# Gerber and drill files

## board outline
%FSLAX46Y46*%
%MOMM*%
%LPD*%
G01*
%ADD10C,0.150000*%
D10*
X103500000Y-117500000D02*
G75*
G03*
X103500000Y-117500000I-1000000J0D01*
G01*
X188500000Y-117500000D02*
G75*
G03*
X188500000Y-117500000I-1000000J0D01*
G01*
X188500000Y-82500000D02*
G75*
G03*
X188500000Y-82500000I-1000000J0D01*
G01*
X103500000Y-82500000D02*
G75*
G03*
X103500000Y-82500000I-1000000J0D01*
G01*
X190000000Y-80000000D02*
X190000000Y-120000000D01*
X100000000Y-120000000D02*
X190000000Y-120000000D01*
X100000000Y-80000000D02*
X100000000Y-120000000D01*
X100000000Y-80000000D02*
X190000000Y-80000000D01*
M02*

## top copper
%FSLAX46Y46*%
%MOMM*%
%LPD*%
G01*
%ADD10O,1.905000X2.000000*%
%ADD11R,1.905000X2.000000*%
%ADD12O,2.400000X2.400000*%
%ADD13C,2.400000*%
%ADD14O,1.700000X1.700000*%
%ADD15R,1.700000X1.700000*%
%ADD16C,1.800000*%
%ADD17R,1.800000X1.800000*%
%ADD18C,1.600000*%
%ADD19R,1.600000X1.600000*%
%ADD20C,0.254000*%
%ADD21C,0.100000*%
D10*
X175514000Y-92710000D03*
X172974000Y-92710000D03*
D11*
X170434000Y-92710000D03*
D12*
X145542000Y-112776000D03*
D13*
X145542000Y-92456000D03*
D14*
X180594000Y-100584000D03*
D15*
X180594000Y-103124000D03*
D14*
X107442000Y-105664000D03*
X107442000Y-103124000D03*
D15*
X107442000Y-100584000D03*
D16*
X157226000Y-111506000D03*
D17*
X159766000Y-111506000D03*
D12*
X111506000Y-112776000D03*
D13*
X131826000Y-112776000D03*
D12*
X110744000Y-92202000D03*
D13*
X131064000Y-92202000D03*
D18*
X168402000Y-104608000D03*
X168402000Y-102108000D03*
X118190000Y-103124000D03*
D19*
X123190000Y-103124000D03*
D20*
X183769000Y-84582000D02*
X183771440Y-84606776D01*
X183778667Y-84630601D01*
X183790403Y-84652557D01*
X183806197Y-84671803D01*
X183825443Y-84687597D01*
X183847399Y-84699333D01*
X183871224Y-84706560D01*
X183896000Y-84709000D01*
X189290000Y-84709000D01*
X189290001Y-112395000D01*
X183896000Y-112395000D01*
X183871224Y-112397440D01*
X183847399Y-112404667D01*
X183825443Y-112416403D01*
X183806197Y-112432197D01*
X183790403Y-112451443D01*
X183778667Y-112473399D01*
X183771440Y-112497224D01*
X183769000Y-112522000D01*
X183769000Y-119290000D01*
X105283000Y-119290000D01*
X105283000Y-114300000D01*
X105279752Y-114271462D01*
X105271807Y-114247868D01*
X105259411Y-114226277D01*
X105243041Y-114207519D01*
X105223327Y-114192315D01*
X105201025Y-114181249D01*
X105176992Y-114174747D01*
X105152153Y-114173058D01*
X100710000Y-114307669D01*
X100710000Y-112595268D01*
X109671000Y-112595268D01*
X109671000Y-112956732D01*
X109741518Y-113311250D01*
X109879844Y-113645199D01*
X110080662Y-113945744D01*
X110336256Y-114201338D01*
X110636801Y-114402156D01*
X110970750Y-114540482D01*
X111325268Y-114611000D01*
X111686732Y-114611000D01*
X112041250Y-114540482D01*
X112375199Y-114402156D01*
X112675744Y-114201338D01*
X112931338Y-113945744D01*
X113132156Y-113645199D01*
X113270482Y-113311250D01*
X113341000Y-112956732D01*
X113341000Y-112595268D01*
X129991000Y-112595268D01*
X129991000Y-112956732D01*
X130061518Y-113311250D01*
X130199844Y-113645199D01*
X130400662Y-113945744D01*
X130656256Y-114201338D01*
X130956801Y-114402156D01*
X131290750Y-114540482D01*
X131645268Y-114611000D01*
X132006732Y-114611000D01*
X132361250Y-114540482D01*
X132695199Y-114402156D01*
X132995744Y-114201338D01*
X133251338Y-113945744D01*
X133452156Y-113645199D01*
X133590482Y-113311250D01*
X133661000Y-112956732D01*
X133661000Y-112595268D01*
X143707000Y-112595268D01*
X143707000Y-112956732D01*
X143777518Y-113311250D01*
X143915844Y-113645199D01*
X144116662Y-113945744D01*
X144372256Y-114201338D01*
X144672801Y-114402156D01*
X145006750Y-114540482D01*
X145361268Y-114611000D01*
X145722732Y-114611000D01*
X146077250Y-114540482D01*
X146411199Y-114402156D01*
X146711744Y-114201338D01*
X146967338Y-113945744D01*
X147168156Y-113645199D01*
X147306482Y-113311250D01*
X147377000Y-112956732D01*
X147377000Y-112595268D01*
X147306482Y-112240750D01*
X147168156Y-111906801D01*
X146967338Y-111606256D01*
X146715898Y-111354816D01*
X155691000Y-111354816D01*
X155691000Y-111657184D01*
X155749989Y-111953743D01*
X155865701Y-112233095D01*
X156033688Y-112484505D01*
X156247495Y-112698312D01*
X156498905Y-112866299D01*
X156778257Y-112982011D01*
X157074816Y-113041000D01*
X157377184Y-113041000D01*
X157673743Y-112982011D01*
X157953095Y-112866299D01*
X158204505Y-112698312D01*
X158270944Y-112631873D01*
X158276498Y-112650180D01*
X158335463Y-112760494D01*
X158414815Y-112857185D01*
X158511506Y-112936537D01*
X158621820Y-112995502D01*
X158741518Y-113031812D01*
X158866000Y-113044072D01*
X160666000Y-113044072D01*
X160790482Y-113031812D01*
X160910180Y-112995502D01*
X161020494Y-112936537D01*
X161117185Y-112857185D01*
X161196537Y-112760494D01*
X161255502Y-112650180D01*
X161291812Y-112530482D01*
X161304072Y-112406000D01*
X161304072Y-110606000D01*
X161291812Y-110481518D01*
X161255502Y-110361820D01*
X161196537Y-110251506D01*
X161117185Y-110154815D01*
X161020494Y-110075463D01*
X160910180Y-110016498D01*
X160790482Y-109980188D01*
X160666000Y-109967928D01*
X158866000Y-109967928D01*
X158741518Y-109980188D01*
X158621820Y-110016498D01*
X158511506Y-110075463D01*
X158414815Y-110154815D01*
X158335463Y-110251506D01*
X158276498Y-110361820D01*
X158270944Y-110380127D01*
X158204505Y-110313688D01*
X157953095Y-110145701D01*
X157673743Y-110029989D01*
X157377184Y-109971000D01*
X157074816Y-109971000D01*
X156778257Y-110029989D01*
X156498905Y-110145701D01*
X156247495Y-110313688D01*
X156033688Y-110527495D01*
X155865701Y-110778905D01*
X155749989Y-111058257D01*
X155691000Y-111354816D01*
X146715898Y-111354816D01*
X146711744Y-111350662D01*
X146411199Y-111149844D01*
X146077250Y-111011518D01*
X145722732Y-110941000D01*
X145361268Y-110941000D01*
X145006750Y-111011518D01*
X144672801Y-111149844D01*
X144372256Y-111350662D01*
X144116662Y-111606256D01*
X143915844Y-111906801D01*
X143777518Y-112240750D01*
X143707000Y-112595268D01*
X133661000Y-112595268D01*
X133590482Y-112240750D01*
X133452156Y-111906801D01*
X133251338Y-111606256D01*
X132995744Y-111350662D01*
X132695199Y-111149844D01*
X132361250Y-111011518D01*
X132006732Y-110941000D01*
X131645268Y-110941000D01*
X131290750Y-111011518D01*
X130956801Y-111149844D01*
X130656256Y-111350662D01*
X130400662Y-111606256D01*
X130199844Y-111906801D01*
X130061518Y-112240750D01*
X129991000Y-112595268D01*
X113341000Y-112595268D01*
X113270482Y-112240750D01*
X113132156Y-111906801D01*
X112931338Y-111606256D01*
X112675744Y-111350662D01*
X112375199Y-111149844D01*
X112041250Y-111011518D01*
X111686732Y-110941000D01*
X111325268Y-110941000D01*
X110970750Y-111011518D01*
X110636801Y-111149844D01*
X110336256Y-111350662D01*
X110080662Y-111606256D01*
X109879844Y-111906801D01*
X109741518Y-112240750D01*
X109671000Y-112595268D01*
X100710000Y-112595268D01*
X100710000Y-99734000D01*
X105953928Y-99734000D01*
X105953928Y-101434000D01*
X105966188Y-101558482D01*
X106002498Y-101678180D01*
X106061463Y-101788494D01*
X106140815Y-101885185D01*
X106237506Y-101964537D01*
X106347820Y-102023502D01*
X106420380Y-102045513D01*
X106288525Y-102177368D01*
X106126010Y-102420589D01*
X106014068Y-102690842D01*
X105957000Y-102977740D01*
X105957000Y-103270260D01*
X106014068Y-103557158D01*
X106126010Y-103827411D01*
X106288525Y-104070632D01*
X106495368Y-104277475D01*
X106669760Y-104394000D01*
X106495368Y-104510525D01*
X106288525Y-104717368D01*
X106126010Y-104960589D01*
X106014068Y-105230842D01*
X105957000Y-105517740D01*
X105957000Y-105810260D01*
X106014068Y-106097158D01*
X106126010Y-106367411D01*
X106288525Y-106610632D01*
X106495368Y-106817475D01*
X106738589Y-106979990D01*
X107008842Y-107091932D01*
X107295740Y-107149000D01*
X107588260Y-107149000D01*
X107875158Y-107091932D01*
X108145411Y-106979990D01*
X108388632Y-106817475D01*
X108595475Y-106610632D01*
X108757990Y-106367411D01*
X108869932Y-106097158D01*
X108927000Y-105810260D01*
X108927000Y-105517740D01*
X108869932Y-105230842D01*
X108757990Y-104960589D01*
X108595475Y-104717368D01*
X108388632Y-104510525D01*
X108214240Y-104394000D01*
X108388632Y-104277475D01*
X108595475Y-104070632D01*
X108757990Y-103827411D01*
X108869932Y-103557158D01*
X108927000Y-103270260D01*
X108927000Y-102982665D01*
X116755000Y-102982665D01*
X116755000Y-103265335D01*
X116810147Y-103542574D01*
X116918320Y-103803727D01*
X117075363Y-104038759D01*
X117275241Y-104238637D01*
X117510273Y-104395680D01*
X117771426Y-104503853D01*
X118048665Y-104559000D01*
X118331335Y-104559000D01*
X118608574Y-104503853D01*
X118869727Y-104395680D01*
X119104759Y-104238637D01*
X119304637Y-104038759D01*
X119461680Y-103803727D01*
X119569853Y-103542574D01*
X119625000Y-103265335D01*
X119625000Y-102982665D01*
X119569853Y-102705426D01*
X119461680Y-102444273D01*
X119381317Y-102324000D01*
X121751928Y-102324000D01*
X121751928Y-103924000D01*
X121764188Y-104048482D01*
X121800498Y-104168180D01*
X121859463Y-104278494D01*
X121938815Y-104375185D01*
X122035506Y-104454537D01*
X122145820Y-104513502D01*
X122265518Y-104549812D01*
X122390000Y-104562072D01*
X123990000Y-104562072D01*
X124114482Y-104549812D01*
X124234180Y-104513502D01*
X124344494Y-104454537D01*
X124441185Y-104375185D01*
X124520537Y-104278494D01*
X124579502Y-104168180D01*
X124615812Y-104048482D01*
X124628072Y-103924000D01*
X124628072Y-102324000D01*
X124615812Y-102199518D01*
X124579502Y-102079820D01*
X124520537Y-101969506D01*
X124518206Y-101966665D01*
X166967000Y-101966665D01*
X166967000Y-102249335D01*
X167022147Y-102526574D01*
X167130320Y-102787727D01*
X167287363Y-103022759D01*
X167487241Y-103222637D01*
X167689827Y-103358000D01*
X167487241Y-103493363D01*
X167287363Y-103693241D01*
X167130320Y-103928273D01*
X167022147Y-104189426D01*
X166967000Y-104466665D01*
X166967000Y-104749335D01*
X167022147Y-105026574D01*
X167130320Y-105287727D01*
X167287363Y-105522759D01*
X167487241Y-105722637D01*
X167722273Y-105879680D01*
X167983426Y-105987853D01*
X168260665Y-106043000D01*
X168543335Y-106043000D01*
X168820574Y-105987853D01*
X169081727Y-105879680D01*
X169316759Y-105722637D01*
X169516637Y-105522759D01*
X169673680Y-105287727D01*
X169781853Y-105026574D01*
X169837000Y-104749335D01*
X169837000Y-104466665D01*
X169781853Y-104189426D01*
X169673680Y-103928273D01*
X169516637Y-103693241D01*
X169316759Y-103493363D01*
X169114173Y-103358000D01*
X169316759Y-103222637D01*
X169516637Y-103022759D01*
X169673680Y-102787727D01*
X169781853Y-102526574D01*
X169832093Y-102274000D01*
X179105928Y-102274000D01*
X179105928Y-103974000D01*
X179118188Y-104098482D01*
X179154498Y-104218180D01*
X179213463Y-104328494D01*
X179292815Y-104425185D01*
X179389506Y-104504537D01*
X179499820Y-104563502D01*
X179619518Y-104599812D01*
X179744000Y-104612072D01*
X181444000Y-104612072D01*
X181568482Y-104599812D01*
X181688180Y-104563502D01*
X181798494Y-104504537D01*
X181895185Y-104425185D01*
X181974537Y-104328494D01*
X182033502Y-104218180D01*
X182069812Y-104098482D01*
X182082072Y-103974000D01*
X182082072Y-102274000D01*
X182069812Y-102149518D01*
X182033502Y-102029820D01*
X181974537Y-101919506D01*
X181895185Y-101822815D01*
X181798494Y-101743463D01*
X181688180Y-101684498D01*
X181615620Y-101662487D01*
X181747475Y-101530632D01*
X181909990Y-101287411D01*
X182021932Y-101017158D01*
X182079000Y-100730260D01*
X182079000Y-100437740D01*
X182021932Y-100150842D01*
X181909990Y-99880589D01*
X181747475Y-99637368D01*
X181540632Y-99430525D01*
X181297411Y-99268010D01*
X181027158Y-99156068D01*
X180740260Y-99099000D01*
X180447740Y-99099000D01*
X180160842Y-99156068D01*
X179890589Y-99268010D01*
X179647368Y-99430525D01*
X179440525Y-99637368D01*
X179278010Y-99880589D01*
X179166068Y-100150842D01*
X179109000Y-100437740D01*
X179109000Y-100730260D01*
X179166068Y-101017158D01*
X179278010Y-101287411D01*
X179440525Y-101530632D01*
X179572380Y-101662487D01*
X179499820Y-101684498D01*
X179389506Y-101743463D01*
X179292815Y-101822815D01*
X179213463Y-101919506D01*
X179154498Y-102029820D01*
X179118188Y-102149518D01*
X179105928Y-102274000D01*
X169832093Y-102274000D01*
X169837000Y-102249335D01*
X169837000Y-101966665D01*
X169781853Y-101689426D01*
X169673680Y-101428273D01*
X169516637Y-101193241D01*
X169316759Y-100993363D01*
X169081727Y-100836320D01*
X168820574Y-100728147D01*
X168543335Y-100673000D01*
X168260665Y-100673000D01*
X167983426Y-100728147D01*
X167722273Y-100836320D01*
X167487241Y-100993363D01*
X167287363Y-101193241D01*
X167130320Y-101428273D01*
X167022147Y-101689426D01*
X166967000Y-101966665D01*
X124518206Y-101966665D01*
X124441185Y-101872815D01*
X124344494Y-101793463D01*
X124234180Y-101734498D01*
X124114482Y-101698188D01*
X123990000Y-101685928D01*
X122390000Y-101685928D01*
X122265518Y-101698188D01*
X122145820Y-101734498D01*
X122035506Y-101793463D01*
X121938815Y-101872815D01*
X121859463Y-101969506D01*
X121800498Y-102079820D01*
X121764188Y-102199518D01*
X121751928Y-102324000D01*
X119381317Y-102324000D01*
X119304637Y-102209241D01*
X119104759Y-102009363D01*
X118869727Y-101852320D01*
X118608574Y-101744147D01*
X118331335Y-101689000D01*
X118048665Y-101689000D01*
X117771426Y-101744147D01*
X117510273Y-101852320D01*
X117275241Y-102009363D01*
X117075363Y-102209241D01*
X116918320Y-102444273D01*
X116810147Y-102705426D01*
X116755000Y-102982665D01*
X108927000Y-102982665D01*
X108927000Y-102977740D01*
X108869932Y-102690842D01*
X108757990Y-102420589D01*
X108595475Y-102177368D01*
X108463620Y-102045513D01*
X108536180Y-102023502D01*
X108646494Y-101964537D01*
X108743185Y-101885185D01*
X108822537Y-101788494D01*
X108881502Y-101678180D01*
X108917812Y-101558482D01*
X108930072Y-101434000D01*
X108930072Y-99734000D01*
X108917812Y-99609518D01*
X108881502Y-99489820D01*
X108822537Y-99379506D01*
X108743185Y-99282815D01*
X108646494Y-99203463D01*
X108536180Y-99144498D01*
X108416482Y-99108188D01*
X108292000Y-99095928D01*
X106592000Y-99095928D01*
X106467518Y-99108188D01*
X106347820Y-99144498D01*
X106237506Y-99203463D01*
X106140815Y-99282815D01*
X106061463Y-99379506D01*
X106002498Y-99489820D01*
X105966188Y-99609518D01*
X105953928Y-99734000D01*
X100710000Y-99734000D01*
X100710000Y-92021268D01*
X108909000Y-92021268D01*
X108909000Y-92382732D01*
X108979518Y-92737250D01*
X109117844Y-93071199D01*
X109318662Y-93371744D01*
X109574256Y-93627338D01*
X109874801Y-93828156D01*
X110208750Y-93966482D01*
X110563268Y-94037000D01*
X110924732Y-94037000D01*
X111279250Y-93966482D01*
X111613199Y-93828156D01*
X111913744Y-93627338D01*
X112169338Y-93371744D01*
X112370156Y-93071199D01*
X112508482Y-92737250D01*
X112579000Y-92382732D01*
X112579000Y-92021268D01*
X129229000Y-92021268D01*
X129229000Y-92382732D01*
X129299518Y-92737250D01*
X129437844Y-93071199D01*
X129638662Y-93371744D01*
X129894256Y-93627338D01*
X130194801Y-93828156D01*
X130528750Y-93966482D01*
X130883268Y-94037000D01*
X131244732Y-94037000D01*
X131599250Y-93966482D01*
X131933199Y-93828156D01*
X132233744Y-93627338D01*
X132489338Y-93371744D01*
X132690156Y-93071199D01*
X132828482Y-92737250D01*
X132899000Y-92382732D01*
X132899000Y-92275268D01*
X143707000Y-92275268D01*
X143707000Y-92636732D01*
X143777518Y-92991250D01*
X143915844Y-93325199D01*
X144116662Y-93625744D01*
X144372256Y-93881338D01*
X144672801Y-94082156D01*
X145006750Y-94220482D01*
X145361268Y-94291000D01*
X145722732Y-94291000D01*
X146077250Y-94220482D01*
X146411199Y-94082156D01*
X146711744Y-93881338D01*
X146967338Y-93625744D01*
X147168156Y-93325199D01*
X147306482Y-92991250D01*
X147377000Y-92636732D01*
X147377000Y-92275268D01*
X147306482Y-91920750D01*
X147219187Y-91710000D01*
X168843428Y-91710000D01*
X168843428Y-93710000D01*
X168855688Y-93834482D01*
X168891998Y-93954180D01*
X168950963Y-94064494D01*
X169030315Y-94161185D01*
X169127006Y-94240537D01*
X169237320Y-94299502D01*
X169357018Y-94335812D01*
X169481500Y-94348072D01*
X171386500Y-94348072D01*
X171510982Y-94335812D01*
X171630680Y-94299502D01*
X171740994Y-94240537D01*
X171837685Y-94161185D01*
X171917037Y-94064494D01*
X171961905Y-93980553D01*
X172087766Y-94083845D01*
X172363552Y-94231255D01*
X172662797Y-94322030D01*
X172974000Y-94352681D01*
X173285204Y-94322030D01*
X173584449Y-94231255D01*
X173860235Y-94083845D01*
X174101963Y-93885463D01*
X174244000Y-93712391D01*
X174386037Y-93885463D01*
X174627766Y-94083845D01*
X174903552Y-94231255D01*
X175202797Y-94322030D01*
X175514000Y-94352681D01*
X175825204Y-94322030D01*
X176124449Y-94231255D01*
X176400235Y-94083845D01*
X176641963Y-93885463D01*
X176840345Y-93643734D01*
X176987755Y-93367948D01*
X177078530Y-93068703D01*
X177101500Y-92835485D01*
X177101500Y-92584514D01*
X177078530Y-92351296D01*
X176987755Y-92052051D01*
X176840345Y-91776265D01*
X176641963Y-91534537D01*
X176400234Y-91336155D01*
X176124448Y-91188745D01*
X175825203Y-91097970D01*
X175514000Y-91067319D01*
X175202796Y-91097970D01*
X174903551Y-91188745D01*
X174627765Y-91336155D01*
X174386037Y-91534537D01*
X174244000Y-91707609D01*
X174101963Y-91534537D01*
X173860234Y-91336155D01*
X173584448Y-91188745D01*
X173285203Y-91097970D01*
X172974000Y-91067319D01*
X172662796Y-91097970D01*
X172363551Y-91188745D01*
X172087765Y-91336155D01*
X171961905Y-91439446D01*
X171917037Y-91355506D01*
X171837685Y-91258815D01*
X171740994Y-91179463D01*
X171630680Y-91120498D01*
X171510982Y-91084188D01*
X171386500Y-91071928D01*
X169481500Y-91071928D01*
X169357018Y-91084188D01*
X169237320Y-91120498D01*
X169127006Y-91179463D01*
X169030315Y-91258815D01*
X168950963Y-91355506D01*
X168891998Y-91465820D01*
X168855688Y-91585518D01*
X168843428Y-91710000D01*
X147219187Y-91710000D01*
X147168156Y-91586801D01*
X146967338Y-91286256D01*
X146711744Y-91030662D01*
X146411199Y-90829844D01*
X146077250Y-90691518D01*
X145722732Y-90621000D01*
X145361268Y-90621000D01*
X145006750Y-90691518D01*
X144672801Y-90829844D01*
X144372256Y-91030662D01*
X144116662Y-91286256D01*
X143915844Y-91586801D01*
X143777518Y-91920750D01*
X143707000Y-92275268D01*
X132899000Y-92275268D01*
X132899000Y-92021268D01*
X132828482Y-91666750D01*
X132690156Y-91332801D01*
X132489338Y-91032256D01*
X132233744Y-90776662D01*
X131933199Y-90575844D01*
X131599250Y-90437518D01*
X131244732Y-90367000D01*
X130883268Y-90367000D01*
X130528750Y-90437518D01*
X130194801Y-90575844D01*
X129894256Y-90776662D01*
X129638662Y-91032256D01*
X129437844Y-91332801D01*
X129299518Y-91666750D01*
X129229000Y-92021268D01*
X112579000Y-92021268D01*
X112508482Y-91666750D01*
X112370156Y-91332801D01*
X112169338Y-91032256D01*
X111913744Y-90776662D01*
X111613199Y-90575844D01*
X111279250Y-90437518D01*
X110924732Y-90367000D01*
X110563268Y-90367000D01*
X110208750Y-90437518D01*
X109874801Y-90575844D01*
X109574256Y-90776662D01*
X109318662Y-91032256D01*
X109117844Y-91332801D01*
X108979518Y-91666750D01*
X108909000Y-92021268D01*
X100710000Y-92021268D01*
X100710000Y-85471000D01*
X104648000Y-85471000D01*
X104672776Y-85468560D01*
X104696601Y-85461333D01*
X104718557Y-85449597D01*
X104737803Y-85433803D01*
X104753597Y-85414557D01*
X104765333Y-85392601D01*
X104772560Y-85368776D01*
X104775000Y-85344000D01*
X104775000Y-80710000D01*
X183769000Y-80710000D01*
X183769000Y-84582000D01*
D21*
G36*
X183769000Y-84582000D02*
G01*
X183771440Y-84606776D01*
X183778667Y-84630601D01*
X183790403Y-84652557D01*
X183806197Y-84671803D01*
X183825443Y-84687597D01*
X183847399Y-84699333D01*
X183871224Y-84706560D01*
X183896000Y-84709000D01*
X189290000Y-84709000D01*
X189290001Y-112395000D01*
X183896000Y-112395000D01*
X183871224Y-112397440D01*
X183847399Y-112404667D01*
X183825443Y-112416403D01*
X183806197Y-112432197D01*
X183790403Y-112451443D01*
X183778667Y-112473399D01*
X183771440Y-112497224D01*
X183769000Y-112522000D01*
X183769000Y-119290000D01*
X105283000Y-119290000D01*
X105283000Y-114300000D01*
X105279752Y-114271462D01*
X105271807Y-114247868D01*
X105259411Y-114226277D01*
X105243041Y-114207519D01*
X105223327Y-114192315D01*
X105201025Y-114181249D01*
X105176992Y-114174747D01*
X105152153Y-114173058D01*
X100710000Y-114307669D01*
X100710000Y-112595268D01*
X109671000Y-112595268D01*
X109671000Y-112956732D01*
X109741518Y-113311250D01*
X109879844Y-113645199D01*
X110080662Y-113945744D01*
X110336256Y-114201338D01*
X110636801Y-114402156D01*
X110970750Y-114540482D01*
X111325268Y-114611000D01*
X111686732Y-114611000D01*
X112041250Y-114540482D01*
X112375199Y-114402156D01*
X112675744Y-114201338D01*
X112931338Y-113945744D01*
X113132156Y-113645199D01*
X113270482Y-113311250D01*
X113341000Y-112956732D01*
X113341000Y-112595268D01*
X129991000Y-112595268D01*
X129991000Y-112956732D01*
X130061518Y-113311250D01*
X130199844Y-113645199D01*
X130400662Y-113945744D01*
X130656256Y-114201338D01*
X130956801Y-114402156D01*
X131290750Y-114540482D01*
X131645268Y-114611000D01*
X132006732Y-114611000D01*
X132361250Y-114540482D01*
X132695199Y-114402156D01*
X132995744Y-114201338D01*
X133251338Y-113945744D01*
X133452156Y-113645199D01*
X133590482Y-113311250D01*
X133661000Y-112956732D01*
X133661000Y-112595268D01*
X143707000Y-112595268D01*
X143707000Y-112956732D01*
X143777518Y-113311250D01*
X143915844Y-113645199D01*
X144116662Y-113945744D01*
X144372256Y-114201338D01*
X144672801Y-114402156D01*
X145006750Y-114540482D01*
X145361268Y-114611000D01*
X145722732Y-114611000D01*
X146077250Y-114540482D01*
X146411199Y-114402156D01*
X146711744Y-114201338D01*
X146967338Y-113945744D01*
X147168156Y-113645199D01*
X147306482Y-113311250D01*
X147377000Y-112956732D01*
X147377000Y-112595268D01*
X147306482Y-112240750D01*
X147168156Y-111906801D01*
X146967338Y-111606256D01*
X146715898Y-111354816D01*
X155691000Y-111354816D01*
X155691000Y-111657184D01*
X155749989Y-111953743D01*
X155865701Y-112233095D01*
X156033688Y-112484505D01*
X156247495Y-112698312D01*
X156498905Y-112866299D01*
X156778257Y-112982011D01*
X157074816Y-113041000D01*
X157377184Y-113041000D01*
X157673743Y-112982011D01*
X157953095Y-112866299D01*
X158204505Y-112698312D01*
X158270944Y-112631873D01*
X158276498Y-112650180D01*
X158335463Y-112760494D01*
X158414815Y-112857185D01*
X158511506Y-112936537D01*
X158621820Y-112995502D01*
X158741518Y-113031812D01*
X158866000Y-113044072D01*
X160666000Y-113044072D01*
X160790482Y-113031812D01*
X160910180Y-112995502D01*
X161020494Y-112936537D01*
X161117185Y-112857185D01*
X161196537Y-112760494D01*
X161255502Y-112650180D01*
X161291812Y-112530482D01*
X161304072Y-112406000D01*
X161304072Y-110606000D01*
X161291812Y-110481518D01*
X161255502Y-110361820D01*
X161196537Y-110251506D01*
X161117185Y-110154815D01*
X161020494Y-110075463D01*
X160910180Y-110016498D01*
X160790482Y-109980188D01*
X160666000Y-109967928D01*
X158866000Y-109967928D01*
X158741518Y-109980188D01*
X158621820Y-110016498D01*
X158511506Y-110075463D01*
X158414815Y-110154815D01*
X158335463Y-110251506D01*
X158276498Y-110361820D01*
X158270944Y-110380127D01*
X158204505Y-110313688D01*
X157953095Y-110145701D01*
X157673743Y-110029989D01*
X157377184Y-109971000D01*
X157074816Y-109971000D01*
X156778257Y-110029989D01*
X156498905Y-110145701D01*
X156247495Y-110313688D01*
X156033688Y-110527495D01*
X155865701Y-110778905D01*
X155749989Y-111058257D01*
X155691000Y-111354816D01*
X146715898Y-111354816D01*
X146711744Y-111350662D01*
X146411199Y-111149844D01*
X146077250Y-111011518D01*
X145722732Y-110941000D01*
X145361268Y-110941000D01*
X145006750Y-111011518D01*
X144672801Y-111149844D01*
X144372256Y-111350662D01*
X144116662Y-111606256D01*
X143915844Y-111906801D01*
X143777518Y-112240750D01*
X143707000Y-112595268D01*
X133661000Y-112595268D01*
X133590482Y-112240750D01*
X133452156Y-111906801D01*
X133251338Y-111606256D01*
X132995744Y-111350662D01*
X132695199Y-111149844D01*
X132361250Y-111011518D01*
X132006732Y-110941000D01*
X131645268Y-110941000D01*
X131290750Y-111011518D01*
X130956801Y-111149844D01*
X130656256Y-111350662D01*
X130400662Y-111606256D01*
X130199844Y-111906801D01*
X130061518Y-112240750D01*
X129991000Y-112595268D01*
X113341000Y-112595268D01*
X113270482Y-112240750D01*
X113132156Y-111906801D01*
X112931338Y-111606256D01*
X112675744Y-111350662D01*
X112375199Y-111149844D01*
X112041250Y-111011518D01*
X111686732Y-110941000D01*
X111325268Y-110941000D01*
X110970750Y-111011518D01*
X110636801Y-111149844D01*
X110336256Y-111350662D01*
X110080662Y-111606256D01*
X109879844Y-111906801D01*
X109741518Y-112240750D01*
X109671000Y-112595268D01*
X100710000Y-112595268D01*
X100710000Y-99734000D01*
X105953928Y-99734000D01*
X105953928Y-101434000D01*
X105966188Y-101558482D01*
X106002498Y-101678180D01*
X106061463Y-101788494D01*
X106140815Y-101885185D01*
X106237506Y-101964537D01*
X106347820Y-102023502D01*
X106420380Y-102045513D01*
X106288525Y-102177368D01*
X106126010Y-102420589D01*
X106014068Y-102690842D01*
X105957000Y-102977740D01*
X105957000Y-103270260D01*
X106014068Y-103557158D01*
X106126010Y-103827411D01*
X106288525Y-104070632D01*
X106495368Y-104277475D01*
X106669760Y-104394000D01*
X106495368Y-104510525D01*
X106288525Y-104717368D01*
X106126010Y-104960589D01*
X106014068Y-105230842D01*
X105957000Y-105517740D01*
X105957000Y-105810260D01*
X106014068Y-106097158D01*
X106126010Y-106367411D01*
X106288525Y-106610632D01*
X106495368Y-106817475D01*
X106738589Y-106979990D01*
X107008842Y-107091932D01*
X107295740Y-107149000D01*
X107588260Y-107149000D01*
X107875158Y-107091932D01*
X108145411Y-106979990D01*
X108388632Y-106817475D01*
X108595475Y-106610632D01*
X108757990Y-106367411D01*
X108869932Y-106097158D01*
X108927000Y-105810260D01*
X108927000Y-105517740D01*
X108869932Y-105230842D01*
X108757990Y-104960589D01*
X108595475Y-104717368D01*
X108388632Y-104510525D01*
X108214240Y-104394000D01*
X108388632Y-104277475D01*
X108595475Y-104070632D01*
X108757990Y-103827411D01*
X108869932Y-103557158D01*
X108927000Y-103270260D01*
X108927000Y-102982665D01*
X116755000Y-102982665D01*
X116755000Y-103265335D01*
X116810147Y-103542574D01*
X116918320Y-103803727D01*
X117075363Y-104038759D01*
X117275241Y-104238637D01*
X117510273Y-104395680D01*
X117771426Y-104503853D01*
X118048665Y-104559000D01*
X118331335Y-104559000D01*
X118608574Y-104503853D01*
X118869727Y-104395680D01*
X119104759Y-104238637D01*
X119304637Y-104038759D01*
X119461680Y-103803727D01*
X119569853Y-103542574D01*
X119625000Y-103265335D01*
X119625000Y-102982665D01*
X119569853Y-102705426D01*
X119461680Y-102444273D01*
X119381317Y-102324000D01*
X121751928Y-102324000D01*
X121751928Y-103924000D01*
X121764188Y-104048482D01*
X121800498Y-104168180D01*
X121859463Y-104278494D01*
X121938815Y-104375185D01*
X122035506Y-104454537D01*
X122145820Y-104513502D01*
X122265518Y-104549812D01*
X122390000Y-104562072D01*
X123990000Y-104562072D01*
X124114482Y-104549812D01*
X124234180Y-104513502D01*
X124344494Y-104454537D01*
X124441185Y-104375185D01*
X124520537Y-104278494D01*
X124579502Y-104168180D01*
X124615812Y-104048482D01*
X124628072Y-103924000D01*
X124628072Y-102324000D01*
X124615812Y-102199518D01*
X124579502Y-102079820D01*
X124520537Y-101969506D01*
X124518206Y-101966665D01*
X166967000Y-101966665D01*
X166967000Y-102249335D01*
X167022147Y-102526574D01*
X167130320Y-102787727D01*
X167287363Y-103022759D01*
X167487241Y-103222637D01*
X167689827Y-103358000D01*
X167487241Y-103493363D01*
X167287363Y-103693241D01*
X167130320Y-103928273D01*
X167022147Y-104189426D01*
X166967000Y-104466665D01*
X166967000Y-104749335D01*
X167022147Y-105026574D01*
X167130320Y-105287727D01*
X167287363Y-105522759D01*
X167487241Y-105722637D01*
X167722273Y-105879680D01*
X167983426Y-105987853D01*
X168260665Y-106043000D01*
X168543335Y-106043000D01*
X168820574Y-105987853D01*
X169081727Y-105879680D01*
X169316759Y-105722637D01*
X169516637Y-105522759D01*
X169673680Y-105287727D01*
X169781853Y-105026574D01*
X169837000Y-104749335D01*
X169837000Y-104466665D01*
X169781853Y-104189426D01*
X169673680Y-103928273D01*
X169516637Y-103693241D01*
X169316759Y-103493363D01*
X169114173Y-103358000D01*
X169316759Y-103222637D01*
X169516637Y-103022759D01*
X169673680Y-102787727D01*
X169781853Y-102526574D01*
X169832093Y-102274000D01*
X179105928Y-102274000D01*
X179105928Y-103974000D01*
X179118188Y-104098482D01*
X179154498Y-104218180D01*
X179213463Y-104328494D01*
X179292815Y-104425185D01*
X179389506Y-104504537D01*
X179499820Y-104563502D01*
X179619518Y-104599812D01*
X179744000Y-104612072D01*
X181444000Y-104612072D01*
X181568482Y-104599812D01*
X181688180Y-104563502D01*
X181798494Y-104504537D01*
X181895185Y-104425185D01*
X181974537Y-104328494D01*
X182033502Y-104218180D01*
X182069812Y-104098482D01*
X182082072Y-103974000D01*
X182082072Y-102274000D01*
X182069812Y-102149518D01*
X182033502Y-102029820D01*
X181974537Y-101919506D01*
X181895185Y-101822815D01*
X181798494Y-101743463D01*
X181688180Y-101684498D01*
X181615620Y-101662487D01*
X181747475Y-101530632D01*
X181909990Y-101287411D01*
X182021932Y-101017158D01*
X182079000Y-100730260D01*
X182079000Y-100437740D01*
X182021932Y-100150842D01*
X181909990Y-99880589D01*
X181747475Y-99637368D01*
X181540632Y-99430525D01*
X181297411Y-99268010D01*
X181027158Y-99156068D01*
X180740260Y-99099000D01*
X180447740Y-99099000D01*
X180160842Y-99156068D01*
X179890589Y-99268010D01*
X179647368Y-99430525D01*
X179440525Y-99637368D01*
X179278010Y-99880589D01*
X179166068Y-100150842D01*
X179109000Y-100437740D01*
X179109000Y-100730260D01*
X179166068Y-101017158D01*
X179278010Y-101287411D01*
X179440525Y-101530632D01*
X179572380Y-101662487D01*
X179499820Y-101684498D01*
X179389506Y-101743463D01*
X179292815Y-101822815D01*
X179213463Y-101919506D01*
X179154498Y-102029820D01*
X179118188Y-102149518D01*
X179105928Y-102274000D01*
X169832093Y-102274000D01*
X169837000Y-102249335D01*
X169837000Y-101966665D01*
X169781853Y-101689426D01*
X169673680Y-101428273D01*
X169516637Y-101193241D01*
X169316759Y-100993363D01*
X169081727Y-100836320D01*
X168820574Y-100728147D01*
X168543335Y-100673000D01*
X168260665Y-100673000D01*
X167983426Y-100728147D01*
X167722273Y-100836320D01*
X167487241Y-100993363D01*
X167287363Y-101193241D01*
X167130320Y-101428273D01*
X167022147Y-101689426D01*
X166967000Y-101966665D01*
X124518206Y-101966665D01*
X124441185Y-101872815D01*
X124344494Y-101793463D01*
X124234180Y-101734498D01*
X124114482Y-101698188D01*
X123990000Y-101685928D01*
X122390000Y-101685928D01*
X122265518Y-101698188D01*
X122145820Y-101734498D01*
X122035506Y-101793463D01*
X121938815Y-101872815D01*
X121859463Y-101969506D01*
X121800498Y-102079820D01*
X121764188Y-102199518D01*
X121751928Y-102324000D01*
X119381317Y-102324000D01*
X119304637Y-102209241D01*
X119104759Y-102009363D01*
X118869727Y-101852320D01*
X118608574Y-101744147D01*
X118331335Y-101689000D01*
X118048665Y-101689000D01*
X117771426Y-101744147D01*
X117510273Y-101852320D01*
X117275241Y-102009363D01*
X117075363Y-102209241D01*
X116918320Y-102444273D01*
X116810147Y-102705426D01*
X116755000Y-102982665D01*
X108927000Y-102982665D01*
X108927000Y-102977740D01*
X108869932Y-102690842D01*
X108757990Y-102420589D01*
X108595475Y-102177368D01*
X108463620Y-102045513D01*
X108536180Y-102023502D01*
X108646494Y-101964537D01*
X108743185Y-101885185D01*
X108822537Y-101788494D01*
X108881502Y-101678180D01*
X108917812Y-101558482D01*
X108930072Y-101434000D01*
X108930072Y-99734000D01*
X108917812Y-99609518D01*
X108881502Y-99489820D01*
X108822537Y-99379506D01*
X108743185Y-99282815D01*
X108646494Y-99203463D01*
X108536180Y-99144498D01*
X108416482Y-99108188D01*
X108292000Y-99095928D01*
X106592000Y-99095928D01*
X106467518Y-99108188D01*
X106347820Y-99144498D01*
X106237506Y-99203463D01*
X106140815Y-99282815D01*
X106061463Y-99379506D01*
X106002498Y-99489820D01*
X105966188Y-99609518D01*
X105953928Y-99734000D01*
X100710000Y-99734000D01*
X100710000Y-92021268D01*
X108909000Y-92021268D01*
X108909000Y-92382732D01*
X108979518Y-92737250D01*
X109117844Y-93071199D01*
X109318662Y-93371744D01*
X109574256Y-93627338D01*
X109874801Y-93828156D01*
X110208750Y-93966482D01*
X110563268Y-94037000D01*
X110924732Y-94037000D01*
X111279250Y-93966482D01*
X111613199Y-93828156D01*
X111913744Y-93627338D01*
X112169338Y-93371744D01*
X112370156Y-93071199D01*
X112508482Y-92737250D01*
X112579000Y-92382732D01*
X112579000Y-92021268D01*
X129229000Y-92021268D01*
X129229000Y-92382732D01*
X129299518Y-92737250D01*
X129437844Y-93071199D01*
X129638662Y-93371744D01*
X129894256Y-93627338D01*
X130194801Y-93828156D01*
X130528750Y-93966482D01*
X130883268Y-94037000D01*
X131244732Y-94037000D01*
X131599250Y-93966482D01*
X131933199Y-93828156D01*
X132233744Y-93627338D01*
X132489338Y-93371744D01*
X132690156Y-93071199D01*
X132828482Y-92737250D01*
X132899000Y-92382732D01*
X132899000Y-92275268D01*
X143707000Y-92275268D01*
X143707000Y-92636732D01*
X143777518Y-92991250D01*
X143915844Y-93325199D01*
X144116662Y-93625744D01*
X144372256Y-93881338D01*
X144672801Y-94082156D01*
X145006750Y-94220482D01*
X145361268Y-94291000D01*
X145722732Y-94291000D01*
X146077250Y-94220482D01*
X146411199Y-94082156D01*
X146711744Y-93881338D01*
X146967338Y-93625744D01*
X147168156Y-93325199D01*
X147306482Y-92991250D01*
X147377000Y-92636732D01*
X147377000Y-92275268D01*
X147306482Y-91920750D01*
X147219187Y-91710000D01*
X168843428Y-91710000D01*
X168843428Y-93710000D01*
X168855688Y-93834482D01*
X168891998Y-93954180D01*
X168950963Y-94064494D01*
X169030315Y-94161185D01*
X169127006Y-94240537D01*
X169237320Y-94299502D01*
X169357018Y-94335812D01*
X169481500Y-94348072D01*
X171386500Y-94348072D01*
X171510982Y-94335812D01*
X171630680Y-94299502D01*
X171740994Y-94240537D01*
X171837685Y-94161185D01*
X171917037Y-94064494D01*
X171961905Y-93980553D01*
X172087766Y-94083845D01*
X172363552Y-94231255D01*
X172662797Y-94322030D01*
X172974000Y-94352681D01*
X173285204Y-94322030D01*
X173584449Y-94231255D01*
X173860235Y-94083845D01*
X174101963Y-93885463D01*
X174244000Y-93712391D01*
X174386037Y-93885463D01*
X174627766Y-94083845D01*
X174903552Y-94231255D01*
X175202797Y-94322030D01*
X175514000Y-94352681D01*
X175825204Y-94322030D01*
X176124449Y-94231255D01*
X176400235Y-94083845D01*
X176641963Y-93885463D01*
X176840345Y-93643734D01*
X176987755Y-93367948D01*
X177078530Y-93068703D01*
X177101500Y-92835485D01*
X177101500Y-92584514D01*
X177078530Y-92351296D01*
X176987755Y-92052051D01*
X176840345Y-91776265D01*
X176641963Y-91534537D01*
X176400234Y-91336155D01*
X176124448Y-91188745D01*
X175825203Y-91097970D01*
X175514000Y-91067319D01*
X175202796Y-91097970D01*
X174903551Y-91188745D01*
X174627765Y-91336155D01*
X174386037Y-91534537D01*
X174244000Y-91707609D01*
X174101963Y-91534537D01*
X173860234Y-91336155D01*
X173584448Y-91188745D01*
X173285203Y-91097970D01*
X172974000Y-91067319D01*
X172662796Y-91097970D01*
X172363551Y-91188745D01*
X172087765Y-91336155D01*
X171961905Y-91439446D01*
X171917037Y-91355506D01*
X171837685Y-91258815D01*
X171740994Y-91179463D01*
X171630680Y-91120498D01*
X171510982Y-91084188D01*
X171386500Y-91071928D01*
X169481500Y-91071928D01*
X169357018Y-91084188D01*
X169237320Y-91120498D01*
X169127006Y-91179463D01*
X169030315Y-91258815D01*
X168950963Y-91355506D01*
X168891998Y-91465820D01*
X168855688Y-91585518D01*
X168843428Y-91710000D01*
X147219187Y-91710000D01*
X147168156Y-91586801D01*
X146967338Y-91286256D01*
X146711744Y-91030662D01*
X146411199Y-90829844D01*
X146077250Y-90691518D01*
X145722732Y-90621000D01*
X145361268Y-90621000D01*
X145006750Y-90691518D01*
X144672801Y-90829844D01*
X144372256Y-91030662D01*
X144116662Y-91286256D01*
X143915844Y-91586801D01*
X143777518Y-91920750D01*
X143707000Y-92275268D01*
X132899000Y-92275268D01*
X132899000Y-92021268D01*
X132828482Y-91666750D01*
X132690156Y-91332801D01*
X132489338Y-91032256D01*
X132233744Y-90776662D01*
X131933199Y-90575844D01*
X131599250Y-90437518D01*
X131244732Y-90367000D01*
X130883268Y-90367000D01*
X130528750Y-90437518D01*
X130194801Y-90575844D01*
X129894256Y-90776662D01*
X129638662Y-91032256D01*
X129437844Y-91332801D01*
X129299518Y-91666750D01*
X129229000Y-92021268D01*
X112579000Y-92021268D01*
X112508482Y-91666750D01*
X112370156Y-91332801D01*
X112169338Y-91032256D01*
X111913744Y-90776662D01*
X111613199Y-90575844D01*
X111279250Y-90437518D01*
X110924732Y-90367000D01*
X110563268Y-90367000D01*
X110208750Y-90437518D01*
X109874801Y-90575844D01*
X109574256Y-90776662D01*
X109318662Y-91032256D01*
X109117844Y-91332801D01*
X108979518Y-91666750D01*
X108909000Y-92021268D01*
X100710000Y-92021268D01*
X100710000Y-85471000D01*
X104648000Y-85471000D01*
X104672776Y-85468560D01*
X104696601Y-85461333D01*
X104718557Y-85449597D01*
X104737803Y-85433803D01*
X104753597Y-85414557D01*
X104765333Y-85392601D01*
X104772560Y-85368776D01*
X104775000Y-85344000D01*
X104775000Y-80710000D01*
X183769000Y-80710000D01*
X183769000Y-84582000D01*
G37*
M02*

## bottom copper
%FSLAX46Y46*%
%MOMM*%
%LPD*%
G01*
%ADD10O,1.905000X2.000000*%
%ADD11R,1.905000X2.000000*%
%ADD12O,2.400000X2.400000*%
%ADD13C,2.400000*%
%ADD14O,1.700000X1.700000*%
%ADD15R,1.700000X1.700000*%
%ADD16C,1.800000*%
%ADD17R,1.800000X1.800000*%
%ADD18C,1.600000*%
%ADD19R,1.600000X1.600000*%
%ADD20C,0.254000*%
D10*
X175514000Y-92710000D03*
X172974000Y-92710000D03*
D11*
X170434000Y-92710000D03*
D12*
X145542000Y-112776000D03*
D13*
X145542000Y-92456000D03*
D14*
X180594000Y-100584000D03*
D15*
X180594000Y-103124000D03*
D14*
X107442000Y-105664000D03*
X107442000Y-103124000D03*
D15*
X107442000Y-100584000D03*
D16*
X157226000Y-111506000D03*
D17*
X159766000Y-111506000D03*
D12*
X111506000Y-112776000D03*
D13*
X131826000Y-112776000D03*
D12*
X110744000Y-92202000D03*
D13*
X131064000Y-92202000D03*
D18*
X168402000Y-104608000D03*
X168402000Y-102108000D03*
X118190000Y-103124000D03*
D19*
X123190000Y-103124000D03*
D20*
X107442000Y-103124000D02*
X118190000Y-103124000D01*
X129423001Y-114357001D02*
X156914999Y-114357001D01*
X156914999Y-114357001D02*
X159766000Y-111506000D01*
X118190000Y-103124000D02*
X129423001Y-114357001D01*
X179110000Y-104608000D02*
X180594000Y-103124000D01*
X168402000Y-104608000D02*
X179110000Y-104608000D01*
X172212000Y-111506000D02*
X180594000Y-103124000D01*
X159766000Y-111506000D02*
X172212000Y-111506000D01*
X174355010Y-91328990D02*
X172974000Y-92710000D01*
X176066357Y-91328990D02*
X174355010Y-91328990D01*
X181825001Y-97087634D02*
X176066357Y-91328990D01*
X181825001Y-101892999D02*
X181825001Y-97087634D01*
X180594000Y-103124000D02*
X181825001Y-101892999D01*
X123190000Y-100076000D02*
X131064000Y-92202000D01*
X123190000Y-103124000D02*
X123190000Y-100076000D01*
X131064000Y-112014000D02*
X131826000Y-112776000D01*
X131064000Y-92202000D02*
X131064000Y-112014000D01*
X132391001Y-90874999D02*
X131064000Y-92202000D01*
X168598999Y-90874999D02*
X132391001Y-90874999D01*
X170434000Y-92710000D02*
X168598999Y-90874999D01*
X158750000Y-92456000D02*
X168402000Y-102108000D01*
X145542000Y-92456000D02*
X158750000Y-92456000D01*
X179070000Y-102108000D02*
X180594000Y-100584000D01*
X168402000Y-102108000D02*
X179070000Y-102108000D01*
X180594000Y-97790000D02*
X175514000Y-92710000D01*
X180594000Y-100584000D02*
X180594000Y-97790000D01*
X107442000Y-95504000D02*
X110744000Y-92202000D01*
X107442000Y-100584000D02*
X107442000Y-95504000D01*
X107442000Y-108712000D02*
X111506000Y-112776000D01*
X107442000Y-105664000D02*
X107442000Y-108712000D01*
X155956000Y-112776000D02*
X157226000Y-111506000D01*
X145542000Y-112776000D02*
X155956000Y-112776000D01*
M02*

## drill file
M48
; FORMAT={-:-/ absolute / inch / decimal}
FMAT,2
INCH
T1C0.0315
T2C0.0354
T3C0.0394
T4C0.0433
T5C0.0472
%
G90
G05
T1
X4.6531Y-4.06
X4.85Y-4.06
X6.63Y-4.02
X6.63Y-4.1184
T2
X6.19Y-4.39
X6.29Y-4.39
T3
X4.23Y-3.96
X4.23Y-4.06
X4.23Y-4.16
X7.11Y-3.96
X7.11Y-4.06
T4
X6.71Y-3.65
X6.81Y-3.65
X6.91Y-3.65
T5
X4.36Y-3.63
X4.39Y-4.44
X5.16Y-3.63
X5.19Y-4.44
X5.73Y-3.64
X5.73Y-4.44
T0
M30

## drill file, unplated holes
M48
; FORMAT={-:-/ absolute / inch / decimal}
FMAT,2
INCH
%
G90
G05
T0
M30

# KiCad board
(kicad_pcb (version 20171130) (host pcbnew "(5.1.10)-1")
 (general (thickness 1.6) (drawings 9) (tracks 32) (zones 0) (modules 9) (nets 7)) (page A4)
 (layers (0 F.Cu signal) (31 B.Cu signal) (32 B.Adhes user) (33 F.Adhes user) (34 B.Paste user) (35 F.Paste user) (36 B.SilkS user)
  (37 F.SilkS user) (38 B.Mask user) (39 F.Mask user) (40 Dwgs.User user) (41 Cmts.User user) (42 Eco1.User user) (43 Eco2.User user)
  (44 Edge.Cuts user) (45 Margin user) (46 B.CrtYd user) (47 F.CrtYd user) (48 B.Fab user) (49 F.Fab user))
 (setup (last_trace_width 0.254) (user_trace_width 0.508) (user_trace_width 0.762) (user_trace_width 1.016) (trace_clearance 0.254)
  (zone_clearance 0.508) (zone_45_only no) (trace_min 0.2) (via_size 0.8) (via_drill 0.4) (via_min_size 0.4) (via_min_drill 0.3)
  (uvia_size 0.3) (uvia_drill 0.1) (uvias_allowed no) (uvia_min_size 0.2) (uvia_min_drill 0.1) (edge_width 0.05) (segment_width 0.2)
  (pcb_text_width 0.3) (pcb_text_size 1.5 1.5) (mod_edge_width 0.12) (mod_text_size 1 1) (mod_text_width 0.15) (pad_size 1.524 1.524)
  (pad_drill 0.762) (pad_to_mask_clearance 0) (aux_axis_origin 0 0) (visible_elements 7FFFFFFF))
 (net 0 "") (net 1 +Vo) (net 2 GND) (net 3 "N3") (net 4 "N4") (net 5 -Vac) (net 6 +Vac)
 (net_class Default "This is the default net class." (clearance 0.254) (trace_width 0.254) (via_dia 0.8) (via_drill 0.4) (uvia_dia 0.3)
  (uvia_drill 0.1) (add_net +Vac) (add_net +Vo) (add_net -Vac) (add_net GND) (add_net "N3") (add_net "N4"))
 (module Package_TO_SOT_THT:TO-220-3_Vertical (layer F.Cu) (at 170.434 92.71)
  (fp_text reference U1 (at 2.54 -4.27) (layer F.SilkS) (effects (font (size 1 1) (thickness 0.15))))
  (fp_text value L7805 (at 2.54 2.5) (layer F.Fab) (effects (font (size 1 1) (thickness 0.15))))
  (pad 3 thru_hole oval (at 5.08 0) (size 1.905 2) (drill 1.1) (layers *.Cu *.Mask) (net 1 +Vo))
  (pad 2 thru_hole oval (at 2.54 0) (size 1.905 2) (drill 1.1) (layers *.Cu *.Mask) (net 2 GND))
  (pad 1 thru_hole rect (at 0 0) (size 1.905 2) (drill 1.1) (layers *.Cu *.Mask) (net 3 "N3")))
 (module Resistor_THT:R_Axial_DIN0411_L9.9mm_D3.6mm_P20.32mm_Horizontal (layer F.Cu) (at 145.542 92.456 270)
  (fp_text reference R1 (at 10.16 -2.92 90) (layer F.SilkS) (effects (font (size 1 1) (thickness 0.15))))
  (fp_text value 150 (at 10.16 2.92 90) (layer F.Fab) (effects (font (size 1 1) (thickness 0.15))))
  (pad 2 thru_hole oval (at 20.32 0 270) (size 2.4 2.4) (drill 1.2) (layers *.Cu *.Mask) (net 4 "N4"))
  (pad 1 thru_hole circle (at 0 0 270) (size 2.4 2.4) (drill 1.2) (layers *.Cu *.Mask) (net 1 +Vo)))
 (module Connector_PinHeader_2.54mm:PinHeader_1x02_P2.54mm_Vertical (layer F.Cu) (at 180.594 103.124 180)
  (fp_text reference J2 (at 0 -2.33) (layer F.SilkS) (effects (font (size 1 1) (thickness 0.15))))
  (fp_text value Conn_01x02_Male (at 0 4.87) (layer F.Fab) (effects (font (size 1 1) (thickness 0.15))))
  (pad 2 thru_hole oval (at 0 2.54 180) (size 1.7 1.7) (drill 1) (layers *.Cu *.Mask) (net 1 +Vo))
  (pad 1 thru_hole rect (at 0 0 180) (size 1.7 1.7) (drill 1) (layers *.Cu *.Mask) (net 2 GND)))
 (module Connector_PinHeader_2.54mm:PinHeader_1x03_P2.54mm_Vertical (layer F.Cu) (at 107.442 100.584)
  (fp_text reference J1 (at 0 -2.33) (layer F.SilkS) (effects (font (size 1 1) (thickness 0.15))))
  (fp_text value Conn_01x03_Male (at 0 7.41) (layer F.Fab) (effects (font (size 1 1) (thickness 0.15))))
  (pad 3 thru_hole oval (at 0 5.08) (size 1.7 1.7) (drill 1) (layers *.Cu *.Mask) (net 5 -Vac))
  (pad 2 thru_hole oval (at 0 2.54) (size 1.7 1.7) (drill 1) (layers *.Cu *.Mask) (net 2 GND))
  (pad 1 thru_hole rect (at 0 0) (size 1.7 1.7) (drill 1) (layers *.Cu *.Mask) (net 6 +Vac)))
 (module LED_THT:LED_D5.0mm (layer F.Cu) (at 159.766 111.506 180)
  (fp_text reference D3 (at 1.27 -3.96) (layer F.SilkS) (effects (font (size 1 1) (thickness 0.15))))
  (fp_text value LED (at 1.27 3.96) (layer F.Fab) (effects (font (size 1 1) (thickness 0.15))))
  (pad 2 thru_hole circle (at 2.54 0 180) (size 1.8 1.8) (drill 0.9) (layers *.Cu *.Mask) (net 4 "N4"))
  (pad 1 thru_hole rect (at 0 0 180) (size 1.8 1.8) (drill 0.9) (layers *.Cu *.Mask) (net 2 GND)))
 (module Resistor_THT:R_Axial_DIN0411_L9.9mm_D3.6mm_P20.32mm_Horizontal (layer F.Cu) (at 131.826 112.776 180)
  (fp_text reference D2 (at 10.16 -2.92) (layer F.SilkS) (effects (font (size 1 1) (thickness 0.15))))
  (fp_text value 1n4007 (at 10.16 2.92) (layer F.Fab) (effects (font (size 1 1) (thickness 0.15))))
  (pad 2 thru_hole oval (at 20.32 0 180) (size 2.4 2.4) (drill 1.2) (layers *.Cu *.Mask) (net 5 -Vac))
  (pad 1 thru_hole circle (at 0 0 180) (size 2.4 2.4) (drill 1.2) (layers *.Cu *.Mask) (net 3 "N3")))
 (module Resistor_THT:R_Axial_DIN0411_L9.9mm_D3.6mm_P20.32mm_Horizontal (layer F.Cu) (at 131.064 92.202 180)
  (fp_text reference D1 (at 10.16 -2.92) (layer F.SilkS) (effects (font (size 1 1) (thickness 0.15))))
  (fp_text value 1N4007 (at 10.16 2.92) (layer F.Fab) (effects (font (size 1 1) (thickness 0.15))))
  (pad 2 thru_hole oval (at 20.32 0 180) (size 2.4 2.4) (drill 1.2) (layers *.Cu *.Mask) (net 6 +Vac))
  (pad 1 thru_hole circle (at 0 0 180) (size 2.4 2.4) (drill 1.2) (layers *.Cu *.Mask) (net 3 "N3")))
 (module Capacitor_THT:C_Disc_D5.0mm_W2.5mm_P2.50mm (layer F.Cu) (at 168.402 102.108 270)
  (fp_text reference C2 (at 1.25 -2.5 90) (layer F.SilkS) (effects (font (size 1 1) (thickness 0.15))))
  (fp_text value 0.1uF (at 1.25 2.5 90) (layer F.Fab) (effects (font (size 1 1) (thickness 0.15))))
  (pad 2 thru_hole circle (at 2.5 0 270) (size 1.6 1.6) (drill 0.8) (layers *.Cu *.Mask) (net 2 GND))
  (pad 1 thru_hole circle (at 0 0 270) (size 1.6 1.6) (drill 0.8) (layers *.Cu *.Mask) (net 1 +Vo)))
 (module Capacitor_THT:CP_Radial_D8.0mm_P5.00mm (layer F.Cu) (at 123.19 103.124 180)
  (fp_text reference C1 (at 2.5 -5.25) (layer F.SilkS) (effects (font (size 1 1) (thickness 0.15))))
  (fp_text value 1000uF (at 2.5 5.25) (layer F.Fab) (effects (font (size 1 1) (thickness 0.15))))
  (pad 2 thru_hole circle (at 5 0 180) (size 1.6 1.6) (drill 0.8) (layers *.Cu *.Mask) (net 2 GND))
  (pad 1 thru_hole rect (at 0 0 180) (size 1.6 1.6) (drill 0.8) (layers *.Cu *.Mask) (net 3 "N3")))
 (gr_circle (center 102.5 117.5) (end 103.5 117.5) (layer Edge.Cuts) (width 0.15))
 (gr_circle (center 187.5 117.5) (end 188.5 117.5) (layer Edge.Cuts) (width 0.15))
 (gr_circle (center 187.5 82.5) (end 188.5 82.5) (layer Edge.Cuts) (width 0.15))
 (gr_circle (center 102.5 82.5) (end 103.5 82.5) (layer Edge.Cuts) (width 0.15))
 (gr_line (start 190 80) (end 190 120) (layer Edge.Cuts) (width 0.15))
 (gr_line (start 100 120) (end 190 120) (layer Edge.Cuts) (width 0.15))
 (gr_line (start 100 80) (end 100 120) (layer Edge.Cuts) (width 0.15))
 (gr_line (start 100 80) (end 190 80) (layer Edge.Cuts) (width 0.15))
 (segment (start 107.442 103.124) (end 118.19 103.124) (width 0.254) (layer B.Cu) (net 2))
 (segment (start 129.423001 114.357001) (end 156.914999 114.357001) (width 0.254) (layer B.Cu) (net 2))
 (segment (start 156.914999 114.357001) (end 159.766 111.506) (width 0.254) (layer B.Cu) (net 2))
 (segment (start 118.19 103.124) (end 129.423001 114.357001) (width 0.254) (layer B.Cu) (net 2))
 (segment (start 179.11 104.608) (end 180.594 103.124) (width 0.254) (layer B.Cu) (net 2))
 (segment (start 168.402 104.608) (end 179.11 104.608) (width 0.254) (layer B.Cu) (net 2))
 (segment (start 172.212 111.506) (end 180.594 103.124) (width 0.254) (layer B.Cu) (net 2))
 (segment (start 159.766 111.506) (end 172.212 111.506) (width 0.254) (layer B.Cu) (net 2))
 (segment (start 174.35501 91.32899) (end 172.974 92.71) (width 0.254) (layer B.Cu) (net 2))
 (segment (start 176.066357 91.32899) (end 174.35501 91.32899) (width 0.254) (layer B.Cu) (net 2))
 (segment (start 181.825001 97.087634) (end 176.066357 91.32899) (width 0.254) (layer B.Cu) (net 2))
 (segment (start 181.825001 101.892999) (end 181.825001 97.087634) (width 0.254) (layer B.Cu) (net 2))
 (segment (start 180.594 103.124) (end 181.825001 101.892999) (width 0.254) (layer B.Cu) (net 2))
 (segment (start 123.19 100.076) (end 131.064 92.202) (width 0.254) (layer B.Cu) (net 3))
 (segment (start 123.19 103.124) (end 123.19 100.076) (width 0.254) (layer B.Cu) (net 3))
 (segment (start 131.064 112.014) (end 131.826 112.776) (width 0.254) (layer B.Cu) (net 3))
 (segment (start 131.064 92.202) (end 131.064 112.014) (width 0.254) (layer B.Cu) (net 3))
 (segment (start 132.391001 90.874999) (end 131.064 92.202) (width 0.254) (layer B.Cu) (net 3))
 (segment (start 168.598999 90.874999) (end 132.391001 90.874999) (width 0.254) (layer B.Cu) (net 3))
 (segment (start 170.434 92.71) (end 168.598999 90.874999) (width 0.254) (layer B.Cu) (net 3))
 (segment (start 158.75 92.456) (end 168.402 102.108) (width 0.254) (layer B.Cu) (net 1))
 (segment (start 145.542 92.456) (end 158.75 92.456) (width 0.254) (layer B.Cu) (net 1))
 (segment (start 179.07 102.108) (end 180.594 100.584) (width 0.254) (layer B.Cu) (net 1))
 (segment (start 168.402 102.108) (end 179.07 102.108) (width 0.254) (layer B.Cu) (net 1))
 (segment (start 180.594 97.79) (end 175.514 92.71) (width 0.254) (layer B.Cu) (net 1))
 (segment (start 180.594 100.584) (end 180.594 97.79) (width 0.254) (layer B.Cu) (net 1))
 (segment (start 107.442 95.504) (end 110.744 92.202) (width 0.254) (layer B.Cu) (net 6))
 (segment (start 107.442 100.584) (end 107.442 95.504) (width 0.254) (layer B.Cu) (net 6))
 (segment (start 107.442 108.712) (end 111.506 112.776) (width 0.254) (layer B.Cu) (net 5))
 (segment (start 107.442 105.664) (end 107.442 108.712) (width 0.254) (layer B.Cu) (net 5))
 (segment (start 155.956 112.776) (end 157.226 111.506) (width 0.254) (layer B.Cu) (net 4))
 (segment (start 145.542 112.776) (end 155.956 112.776) (width 0.254) (layer B.Cu) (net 4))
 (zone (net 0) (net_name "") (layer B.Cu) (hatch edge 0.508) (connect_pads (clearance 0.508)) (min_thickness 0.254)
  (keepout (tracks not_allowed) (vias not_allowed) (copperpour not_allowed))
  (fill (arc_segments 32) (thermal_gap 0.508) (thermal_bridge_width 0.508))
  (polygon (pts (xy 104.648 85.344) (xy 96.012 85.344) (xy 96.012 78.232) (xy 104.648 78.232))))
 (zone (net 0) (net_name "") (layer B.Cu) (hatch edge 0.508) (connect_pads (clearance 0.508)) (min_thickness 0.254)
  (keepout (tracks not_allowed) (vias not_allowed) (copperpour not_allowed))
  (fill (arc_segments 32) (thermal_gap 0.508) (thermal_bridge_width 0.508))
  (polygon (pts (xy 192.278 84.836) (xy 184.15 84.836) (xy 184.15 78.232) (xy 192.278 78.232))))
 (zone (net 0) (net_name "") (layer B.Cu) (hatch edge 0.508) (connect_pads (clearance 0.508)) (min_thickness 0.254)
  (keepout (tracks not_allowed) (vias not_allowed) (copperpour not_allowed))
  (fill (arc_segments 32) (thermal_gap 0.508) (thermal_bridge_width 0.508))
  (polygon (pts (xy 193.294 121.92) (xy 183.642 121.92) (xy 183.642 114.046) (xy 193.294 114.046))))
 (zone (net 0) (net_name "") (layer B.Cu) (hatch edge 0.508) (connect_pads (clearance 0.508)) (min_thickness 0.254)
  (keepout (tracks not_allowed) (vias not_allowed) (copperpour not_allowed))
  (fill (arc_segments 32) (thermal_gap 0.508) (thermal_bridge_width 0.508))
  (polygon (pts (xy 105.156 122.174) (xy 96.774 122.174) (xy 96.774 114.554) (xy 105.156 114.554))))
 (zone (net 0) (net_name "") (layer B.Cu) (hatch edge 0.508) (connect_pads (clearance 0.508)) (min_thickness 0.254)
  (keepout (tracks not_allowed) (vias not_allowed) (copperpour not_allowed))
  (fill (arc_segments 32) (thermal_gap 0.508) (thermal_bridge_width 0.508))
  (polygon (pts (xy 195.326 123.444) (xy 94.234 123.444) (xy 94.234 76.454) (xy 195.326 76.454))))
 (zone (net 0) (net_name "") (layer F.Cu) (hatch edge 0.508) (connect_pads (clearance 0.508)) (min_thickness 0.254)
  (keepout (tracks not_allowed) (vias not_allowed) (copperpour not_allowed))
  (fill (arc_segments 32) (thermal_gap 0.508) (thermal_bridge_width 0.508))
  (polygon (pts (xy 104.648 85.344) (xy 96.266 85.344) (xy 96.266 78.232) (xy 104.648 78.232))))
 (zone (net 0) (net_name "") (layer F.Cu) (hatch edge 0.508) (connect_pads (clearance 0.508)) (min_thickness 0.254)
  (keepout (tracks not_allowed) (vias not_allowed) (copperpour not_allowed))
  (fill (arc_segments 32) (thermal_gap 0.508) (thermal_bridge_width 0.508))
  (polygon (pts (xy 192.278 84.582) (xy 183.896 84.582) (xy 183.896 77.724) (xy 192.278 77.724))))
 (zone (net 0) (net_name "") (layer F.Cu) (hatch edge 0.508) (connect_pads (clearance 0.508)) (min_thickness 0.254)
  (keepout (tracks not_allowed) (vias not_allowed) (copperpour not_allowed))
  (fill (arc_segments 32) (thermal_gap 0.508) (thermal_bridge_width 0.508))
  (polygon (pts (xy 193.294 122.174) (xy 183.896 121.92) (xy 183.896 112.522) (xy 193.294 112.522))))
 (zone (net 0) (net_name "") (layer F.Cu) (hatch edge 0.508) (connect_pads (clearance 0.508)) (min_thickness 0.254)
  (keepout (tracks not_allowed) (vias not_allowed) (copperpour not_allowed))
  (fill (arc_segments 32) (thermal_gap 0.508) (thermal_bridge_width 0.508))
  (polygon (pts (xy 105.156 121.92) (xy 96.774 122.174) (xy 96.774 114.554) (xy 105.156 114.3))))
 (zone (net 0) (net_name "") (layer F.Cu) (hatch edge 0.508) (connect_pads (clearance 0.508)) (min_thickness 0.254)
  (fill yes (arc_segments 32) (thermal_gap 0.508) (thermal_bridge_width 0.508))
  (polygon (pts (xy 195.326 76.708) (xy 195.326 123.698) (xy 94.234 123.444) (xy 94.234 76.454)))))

